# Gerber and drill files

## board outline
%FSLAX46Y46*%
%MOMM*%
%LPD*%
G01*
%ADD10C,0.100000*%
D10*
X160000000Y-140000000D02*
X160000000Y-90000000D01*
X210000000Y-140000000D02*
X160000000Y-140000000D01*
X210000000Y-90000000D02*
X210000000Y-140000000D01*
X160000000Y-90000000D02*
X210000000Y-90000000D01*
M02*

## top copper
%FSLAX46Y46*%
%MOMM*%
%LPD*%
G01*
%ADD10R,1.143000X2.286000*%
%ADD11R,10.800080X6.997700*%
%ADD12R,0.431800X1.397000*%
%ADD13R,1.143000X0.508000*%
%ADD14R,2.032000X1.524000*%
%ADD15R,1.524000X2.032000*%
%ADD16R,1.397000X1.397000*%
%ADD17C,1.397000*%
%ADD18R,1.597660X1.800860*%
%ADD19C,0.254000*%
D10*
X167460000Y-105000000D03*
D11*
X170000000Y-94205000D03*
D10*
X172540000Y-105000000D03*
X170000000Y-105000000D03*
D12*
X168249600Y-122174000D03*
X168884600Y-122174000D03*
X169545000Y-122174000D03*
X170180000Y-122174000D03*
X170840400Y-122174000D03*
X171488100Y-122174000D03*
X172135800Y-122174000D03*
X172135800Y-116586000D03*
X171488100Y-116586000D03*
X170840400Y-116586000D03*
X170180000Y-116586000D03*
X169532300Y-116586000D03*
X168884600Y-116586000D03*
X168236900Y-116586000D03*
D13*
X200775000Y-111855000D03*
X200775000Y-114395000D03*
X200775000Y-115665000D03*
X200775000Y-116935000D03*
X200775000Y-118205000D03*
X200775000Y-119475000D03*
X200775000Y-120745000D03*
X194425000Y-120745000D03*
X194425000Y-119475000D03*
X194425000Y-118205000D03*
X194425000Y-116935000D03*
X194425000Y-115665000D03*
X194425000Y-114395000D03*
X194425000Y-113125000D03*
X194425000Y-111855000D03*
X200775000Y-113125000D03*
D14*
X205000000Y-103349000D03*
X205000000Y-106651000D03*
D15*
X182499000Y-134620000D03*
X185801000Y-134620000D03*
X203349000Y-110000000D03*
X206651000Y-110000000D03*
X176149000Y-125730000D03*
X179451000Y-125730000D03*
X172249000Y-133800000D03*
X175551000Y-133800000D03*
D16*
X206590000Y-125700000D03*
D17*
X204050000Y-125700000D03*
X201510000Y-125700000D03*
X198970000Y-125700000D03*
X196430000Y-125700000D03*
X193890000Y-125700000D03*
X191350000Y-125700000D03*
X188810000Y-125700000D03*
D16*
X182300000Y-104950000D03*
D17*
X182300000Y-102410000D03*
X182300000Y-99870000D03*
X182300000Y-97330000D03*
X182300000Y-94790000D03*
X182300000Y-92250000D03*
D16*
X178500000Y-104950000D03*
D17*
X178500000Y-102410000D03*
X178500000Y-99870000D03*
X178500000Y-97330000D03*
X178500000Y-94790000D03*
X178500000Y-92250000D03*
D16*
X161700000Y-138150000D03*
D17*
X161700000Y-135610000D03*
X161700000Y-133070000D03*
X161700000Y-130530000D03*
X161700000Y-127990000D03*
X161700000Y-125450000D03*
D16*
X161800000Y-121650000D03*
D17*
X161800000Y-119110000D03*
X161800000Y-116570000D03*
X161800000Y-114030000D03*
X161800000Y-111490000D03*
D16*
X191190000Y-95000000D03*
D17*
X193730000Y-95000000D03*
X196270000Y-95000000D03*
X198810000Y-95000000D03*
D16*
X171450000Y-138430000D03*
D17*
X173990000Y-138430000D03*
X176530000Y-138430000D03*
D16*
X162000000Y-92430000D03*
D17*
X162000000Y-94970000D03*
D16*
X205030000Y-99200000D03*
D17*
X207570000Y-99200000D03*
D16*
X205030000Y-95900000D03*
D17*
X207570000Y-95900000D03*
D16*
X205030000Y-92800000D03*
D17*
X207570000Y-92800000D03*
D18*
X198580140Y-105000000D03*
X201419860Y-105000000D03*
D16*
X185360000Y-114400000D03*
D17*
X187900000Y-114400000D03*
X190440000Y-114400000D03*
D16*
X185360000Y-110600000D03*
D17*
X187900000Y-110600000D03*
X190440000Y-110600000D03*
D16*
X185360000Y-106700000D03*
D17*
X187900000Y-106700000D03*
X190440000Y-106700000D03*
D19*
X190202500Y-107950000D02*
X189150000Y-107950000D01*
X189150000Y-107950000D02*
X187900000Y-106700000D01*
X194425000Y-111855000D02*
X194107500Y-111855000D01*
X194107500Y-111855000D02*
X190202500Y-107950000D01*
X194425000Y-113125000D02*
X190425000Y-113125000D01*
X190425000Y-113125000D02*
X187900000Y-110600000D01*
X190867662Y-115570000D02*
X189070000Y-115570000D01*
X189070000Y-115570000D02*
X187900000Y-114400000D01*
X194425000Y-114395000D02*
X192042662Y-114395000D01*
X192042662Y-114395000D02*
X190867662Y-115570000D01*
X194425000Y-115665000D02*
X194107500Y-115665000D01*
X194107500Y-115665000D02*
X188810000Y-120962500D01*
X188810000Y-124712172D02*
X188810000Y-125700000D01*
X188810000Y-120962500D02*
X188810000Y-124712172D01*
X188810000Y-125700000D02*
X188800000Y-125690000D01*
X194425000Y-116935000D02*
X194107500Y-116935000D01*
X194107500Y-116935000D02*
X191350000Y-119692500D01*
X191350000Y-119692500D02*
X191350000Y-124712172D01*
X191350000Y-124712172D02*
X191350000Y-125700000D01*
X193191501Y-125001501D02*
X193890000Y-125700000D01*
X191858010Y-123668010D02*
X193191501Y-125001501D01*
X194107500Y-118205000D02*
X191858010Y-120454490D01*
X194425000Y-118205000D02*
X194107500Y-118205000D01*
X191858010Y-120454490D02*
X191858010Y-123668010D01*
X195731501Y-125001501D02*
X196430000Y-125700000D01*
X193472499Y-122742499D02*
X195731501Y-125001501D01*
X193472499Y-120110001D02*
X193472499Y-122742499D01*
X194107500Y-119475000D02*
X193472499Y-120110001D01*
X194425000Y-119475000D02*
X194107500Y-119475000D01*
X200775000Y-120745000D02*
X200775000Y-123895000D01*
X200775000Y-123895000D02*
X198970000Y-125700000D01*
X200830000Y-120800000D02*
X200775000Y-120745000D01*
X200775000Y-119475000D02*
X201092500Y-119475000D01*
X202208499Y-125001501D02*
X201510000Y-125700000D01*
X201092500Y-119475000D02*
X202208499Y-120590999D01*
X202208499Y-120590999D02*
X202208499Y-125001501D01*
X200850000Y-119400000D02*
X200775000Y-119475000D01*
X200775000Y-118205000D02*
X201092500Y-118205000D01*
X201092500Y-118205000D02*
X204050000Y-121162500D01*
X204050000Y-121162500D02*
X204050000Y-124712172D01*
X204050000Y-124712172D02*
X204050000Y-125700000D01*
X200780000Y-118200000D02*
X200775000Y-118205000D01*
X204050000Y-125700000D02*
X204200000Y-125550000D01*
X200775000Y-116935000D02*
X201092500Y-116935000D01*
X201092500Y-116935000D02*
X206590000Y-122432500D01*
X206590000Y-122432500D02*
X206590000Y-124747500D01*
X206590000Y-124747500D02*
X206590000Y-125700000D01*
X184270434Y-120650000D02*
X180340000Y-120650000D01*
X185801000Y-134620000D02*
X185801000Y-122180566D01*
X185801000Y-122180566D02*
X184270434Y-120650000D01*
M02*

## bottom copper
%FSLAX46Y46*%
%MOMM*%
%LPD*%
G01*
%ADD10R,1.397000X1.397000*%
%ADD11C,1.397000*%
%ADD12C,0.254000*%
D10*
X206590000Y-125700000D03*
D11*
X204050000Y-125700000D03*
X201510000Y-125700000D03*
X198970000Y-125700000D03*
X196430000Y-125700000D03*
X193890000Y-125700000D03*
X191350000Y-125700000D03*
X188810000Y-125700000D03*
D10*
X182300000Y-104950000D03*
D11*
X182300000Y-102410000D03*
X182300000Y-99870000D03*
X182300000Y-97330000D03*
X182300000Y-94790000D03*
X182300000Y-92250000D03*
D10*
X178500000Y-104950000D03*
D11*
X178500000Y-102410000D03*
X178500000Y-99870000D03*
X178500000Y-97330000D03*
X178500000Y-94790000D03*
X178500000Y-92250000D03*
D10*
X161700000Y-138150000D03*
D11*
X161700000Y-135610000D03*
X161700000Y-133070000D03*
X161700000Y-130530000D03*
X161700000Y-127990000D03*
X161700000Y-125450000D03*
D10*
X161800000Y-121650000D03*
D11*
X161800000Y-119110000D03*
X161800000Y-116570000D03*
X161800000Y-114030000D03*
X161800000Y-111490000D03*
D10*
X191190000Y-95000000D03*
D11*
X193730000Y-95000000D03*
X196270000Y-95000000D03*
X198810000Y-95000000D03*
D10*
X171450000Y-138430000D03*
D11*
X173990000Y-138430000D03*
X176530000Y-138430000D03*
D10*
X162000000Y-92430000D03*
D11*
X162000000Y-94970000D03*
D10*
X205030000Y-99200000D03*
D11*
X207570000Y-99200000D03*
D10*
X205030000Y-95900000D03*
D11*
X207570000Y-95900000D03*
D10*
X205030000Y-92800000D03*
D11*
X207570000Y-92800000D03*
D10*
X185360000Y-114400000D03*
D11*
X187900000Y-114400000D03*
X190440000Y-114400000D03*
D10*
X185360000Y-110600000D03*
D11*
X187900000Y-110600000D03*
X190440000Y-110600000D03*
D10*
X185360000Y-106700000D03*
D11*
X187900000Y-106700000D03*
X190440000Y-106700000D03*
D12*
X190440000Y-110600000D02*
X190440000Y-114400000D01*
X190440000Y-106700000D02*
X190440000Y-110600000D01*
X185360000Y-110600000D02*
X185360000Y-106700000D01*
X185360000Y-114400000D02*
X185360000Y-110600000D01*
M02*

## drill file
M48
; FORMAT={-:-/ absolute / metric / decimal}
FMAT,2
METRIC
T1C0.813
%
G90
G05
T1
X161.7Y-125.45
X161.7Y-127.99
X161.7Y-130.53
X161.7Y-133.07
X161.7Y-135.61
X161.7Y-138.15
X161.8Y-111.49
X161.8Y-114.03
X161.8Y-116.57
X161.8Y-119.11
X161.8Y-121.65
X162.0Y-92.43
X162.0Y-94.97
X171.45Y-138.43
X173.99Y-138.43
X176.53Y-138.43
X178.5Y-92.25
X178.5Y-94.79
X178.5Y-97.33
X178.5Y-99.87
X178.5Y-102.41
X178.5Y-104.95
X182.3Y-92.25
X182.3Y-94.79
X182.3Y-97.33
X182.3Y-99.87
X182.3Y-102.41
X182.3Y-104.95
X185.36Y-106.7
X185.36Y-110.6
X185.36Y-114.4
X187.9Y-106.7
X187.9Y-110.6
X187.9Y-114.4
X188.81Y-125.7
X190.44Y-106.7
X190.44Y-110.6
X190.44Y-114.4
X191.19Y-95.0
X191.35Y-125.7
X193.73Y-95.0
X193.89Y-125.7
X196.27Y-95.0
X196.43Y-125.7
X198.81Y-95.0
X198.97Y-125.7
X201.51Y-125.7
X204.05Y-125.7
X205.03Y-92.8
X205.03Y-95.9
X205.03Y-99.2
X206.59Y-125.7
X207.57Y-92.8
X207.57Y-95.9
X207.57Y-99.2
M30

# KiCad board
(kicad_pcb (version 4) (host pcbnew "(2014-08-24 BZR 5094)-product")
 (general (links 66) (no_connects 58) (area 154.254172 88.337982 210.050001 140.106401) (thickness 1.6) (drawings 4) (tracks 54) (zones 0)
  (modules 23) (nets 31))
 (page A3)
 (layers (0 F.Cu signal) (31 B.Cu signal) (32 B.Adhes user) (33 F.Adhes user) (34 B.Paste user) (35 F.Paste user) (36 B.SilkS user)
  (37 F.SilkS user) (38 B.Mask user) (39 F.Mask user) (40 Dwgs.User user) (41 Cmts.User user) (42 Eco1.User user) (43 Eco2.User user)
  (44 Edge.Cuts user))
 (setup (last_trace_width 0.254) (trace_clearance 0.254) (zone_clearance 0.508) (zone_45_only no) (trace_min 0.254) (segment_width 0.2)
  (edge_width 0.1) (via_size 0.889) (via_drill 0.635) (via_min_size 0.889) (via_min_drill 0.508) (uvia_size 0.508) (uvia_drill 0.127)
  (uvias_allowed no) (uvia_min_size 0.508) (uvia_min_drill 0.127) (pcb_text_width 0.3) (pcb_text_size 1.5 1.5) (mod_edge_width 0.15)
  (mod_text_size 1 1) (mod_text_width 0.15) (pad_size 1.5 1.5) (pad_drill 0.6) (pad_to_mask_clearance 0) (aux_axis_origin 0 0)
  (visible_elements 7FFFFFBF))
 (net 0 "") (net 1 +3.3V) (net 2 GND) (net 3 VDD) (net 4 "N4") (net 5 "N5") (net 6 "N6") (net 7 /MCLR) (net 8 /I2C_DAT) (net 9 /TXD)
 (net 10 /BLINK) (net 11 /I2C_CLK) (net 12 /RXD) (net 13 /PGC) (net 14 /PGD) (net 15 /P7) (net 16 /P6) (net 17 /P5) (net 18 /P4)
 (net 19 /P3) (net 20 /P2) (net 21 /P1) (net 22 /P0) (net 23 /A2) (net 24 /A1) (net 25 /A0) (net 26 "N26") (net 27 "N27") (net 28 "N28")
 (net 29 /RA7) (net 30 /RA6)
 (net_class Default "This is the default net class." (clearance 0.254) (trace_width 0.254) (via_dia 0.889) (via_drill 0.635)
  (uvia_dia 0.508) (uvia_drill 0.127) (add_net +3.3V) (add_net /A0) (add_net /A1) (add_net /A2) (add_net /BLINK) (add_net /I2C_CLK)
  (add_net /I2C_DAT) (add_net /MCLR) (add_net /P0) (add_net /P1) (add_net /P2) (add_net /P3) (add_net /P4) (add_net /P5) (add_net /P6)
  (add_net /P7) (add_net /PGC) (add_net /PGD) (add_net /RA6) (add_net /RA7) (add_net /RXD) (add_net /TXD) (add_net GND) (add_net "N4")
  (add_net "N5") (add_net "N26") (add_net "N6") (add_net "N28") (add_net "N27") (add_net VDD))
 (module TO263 (layer F.Cu) (at 170 105)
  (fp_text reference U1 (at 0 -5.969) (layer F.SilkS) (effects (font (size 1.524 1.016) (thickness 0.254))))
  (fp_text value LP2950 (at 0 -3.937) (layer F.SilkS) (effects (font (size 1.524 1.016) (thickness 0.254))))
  (pad 1 smd rect (at -2.54 0) (size 1.143 2.286) (layers F.Cu F.Paste F.Mask) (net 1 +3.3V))
  (pad 2 smd rect (at 0 -10.795) (size 10.80008 6.9977) (layers F.Cu F.Paste F.Mask) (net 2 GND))
  (pad 3 smd rect (at 2.54 0) (size 1.143 2.286) (layers F.Cu F.Paste F.Mask) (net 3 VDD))
  (pad 2 smd rect (at 0 0) (size 1.143 2.286) (layers F.Cu F.Paste F.Mask) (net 2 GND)))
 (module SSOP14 (layer F.Cu) (at 170.18 119.38)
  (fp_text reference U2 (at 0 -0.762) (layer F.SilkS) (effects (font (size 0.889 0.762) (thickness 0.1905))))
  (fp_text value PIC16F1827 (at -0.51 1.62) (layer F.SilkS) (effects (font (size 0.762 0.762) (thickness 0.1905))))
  (pad 1 smd rect (at -1.9304 2.794) (size 0.4318 1.397) (layers F.Cu F.Paste F.Mask) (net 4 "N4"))
  (pad 2 smd rect (at -1.2954 2.794) (size 0.4318 1.397) (layers F.Cu F.Paste F.Mask) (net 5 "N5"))
  (pad 3 smd rect (at -0.635 2.794) (size 0.4318 1.397) (layers F.Cu F.Paste F.Mask) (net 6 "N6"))
  (pad 4 smd rect (at 0 2.794) (size 0.4318 1.397) (layers F.Cu F.Paste F.Mask) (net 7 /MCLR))
  (pad 5 smd rect (at 0.6604 2.794) (size 0.4318 1.397) (layers F.Cu F.Paste F.Mask) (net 2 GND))
  (pad 6 smd rect (at 1.3081 2.794) (size 0.4318 1.397) (layers F.Cu F.Paste F.Mask))
  (pad 7 smd rect (at 1.9558 2.794) (size 0.4318 1.397) (layers F.Cu F.Paste F.Mask) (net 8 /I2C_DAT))
  (pad 8 smd rect (at 1.9558 -2.794) (size 0.4318 1.397) (layers F.Cu F.Paste F.Mask) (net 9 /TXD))
  (pad 9 smd rect (at 1.3081 -2.794) (size 0.4318 1.397) (layers F.Cu F.Paste F.Mask) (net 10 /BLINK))
  (pad 10 smd rect (at 0.6604 -2.794) (size 0.4318 1.397) (layers F.Cu F.Paste F.Mask) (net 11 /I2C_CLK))
  (pad 11 smd rect (at 0 -2.794) (size 0.4318 1.397) (layers F.Cu F.Paste F.Mask) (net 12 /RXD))
  (pad 12 smd rect (at -0.6477 -2.794) (size 0.4318 1.397) (layers F.Cu F.Paste F.Mask) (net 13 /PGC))
  (pad 13 smd rect (at -1.2954 -2.794) (size 0.4318 1.397) (layers F.Cu F.Paste F.Mask) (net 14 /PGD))
  (pad 14 smd rect (at -1.9431 -2.794) (size 0.4318 1.397) (layers F.Cu F.Paste F.Mask) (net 1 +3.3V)))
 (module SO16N (layer F.Cu) (at 197.6 116.3 270)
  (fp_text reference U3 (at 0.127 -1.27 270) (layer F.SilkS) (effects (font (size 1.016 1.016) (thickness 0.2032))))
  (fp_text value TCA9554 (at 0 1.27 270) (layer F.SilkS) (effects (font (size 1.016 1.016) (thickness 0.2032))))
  (pad 16 smd rect (at -4.445 -3.175 270) (size 0.508 1.143) (layers F.Cu F.Paste F.Mask) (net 1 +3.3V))
  (pad 14 smd rect (at -1.905 -3.175 270) (size 0.508 1.143) (layers F.Cu F.Paste F.Mask) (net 11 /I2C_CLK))
  (pad 13 smd rect (at -0.635 -3.175 270) (size 0.508 1.143) (layers F.Cu F.Paste F.Mask))
  (pad 12 smd rect (at 0.635 -3.175 270) (size 0.508 1.143) (layers F.Cu F.Paste F.Mask) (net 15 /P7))
  (pad 11 smd rect (at 1.905 -3.175 270) (size 0.508 1.143) (layers F.Cu F.Paste F.Mask) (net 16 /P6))
  (pad 10 smd rect (at 3.175 -3.175 270) (size 0.508 1.143) (layers F.Cu F.Paste F.Mask) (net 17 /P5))
  (pad 9 smd rect (at 4.445 -3.175 270) (size 0.508 1.143) (layers F.Cu F.Paste F.Mask) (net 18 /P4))
  (pad 8 smd rect (at 4.445 3.175 270) (size 0.508 1.143) (layers F.Cu F.Paste F.Mask) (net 2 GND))
  (pad 7 smd rect (at 3.175 3.175 270) (size 0.508 1.143) (layers F.Cu F.Paste F.Mask) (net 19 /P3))
  (pad 6 smd rect (at 1.905 3.175 270) (size 0.508 1.143) (layers F.Cu F.Paste F.Mask) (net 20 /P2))
  (pad 5 smd rect (at 0.635 3.175 270) (size 0.508 1.143) (layers F.Cu F.Paste F.Mask) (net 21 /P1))
  (pad 4 smd rect (at -0.635 3.175 270) (size 0.508 1.143) (layers F.Cu F.Paste F.Mask) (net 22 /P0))
  (pad 3 smd rect (at -1.905 3.175 270) (size 0.508 1.143) (layers F.Cu F.Paste F.Mask) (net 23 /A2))
  (pad 2 smd rect (at -3.175 3.175 270) (size 0.508 1.143) (layers F.Cu F.Paste F.Mask) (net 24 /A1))
  (pad 1 smd rect (at -4.445 3.175 270) (size 0.508 1.143) (layers F.Cu F.Paste F.Mask) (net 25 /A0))
  (pad 15 smd rect (at -3.175 -3.175 270) (size 0.508 1.143) (layers F.Cu F.Paste F.Mask) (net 8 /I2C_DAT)))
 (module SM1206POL (layer F.Cu) (at 205 105 270)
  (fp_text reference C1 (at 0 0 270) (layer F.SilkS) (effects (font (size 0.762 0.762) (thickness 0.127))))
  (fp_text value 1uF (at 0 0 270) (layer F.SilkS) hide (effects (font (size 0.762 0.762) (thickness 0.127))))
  (pad 1 smd rect (at -1.651 0 270) (size 1.524 2.032) (layers F.Cu F.Paste F.Mask) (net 3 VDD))
  (pad 2 smd rect (at 1.651 0 270) (size 1.524 2.032) (layers F.Cu F.Paste F.Mask) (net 2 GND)))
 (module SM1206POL (layer F.Cu) (at 184.15 134.62)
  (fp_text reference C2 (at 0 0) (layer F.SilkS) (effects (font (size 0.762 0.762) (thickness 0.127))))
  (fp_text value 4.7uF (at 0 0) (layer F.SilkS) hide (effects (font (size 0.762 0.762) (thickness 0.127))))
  (pad 1 smd rect (at -1.651 0) (size 1.524 2.032) (layers F.Cu F.Paste F.Mask) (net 1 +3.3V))
  (pad 2 smd rect (at 1.651 0) (size 1.524 2.032) (layers F.Cu F.Paste F.Mask) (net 2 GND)))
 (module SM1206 (layer F.Cu) (at 205 110)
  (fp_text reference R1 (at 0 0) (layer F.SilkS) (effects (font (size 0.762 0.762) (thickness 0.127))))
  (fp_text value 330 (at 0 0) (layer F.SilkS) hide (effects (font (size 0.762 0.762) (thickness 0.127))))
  (pad 1 smd rect (at -1.651 0) (size 1.524 2.032) (layers F.Cu F.Paste F.Mask) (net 10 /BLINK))
  (pad 2 smd rect (at 1.651 0) (size 1.524 2.032) (layers F.Cu F.Paste F.Mask) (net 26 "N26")))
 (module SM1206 (layer F.Cu) (at 177.8 125.73)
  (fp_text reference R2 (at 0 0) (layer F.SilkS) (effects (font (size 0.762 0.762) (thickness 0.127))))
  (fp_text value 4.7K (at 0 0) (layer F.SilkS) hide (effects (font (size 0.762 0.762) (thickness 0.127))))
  (pad 1 smd rect (at -1.651 0) (size 1.524 2.032) (layers F.Cu F.Paste F.Mask) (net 1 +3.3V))
  (pad 2 smd rect (at 1.651 0) (size 1.524 2.032) (layers F.Cu F.Paste F.Mask) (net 11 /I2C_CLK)))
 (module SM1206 (layer F.Cu) (at 173.9 133.8)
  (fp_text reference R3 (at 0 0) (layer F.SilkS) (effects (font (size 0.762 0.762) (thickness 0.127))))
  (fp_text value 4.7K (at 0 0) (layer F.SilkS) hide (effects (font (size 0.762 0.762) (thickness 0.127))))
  (pad 1 smd rect (at -1.651 0) (size 1.524 2.032) (layers F.Cu F.Paste F.Mask) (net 1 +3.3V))
  (pad 2 smd rect (at 1.651 0) (size 1.524 2.032) (layers F.Cu F.Paste F.Mask) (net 8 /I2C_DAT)))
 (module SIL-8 (layer F.Cu) (at 197.7 125.7 180)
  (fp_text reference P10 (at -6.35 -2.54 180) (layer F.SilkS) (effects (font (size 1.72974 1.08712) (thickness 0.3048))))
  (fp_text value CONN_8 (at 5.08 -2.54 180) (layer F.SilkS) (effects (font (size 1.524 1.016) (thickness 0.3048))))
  (pad 1 thru_hole rect (at -8.89 0 180) (size 1.397 1.397) (drill 0.8128) (layers *.Cu *.Mask F.SilkS) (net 15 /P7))
  (pad 2 thru_hole circle (at -6.35 0 180) (size 1.397 1.397) (drill 0.8128) (layers *.Cu *.Mask F.SilkS) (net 16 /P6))
  (pad 3 thru_hole circle (at -3.81 0 180) (size 1.397 1.397) (drill 0.8128) (layers *.Cu *.Mask F.SilkS) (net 17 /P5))
  (pad 4 thru_hole circle (at -1.27 0 180) (size 1.397 1.397) (drill 0.8128) (layers *.Cu *.Mask F.SilkS) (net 18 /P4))
  (pad 5 thru_hole circle (at 1.27 0 180) (size 1.397 1.397) (drill 0.8128) (layers *.Cu *.Mask F.SilkS) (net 19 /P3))
  (pad 6 thru_hole circle (at 3.81 0 180) (size 1.397 1.397) (drill 0.8128) (layers *.Cu *.Mask F.SilkS) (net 20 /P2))
  (pad 7 thru_hole circle (at 6.35 0 180) (size 1.397 1.397) (drill 0.8128) (layers *.Cu *.Mask F.SilkS) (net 21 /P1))
  (pad 8 thru_hole circle (at 8.89 0 180) (size 1.397 1.397) (drill 0.8128) (layers *.Cu *.Mask F.SilkS) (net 22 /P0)))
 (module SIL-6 (layer F.Cu) (at 182.3 98.6 90)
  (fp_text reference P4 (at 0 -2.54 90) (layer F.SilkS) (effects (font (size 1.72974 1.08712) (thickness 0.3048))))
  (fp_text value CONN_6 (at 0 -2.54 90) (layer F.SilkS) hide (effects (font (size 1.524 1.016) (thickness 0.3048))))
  (pad 1 thru_hole rect (at -6.35 0 90) (size 1.397 1.397) (drill 0.8128) (layers *.Cu *.Mask F.SilkS) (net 1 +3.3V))
  (pad 2 thru_hole circle (at -3.81 0 90) (size 1.397 1.397) (drill 0.8128) (layers *.Cu *.Mask F.SilkS) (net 1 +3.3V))
  (pad 3 thru_hole circle (at -1.27 0 90) (size 1.397 1.397) (drill 0.8128) (layers *.Cu *.Mask F.SilkS) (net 1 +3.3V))
  (pad 4 thru_hole circle (at 1.27 0 90) (size 1.397 1.397) (drill 0.8128) (layers *.Cu *.Mask F.SilkS) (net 1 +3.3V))
  (pad 5 thru_hole circle (at 3.81 0 90) (size 1.397 1.397) (drill 0.8128) (layers *.Cu *.Mask F.SilkS) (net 1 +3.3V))
  (pad 6 thru_hole circle (at 6.35 0 90) (size 1.397 1.397) (drill 0.8128) (layers *.Cu *.Mask F.SilkS) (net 1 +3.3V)))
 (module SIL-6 (layer F.Cu) (at 178.5 98.6 90)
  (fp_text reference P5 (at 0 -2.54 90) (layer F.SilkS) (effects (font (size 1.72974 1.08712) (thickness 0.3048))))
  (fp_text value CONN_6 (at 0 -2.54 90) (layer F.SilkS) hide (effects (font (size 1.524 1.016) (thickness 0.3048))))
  (pad 1 thru_hole rect (at -6.35 0 90) (size 1.397 1.397) (drill 0.8128) (layers *.Cu *.Mask F.SilkS) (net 2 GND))
  (pad 2 thru_hole circle (at -3.81 0 90) (size 1.397 1.397) (drill 0.8128) (layers *.Cu *.Mask F.SilkS) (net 2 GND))
  (pad 3 thru_hole circle (at -1.27 0 90) (size 1.397 1.397) (drill 0.8128) (layers *.Cu *.Mask F.SilkS) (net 2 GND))
  (pad 4 thru_hole circle (at 1.27 0 90) (size 1.397 1.397) (drill 0.8128) (layers *.Cu *.Mask F.SilkS) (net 2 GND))
  (pad 5 thru_hole circle (at 3.81 0 90) (size 1.397 1.397) (drill 0.8128) (layers *.Cu *.Mask F.SilkS) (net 2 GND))
  (pad 6 thru_hole circle (at 6.35 0 90) (size 1.397 1.397) (drill 0.8128) (layers *.Cu *.Mask F.SilkS) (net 2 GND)))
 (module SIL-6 (layer F.Cu) (at 161.7 131.8 90)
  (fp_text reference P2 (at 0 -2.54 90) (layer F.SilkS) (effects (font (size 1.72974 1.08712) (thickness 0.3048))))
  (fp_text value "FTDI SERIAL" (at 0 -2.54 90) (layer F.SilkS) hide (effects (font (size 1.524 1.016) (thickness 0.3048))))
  (pad 1 thru_hole rect (at -6.35 0 90) (size 1.397 1.397) (drill 0.8128) (layers *.Cu *.Mask F.SilkS) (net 2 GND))
  (pad 2 thru_hole circle (at -3.81 0 90) (size 1.397 1.397) (drill 0.8128) (layers *.Cu *.Mask F.SilkS))
  (pad 3 thru_hole circle (at -1.27 0 90) (size 1.397 1.397) (drill 0.8128) (layers *.Cu *.Mask F.SilkS) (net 3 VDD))
  (pad 4 thru_hole circle (at 1.27 0 90) (size 1.397 1.397) (drill 0.8128) (layers *.Cu *.Mask F.SilkS) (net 9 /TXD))
  (pad 5 thru_hole circle (at 3.81 0 90) (size 1.397 1.397) (drill 0.8128) (layers *.Cu *.Mask F.SilkS) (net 12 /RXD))
  (pad 6 thru_hole circle (at 6.35 0 90) (size 1.397 1.397) (drill 0.8128) (layers *.Cu *.Mask F.SilkS)))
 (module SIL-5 (layer F.Cu) (at 161.8 115.3 90)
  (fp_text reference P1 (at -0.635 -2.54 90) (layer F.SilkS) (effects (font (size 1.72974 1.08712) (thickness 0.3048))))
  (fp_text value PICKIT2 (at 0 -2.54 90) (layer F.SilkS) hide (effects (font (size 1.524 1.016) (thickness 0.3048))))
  (pad 1 thru_hole rect (at -6.35 0 90) (size 1.397 1.397) (drill 0.8128) (layers *.Cu *.Mask F.SilkS) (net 13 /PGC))
  (pad 2 thru_hole circle (at -3.81 0 90) (size 1.397 1.397) (drill 0.8128) (layers *.Cu *.Mask F.SilkS) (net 14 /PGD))
  (pad 3 thru_hole circle (at -1.27 0 90) (size 1.397 1.397) (drill 0.8128) (layers *.Cu *.Mask F.SilkS) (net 2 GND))
  (pad 4 thru_hole circle (at 1.27 0 90) (size 1.397 1.397) (drill 0.8128) (layers *.Cu *.Mask F.SilkS) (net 3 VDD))
  (pad 5 thru_hole circle (at 3.81 0 90) (size 1.397 1.397) (drill 0.8128) (layers *.Cu *.Mask F.SilkS) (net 7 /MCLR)))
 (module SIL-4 (layer F.Cu) (at 195 95)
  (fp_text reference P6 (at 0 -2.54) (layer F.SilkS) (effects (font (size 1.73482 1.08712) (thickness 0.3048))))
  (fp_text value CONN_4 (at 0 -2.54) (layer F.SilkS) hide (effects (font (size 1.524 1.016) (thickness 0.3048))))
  (pad 1 thru_hole rect (at -3.81 0) (size 1.397 1.397) (drill 0.8128) (layers *.Cu *.Mask F.SilkS) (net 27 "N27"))
  (pad 2 thru_hole circle (at -1.27 0) (size 1.397 1.397) (drill 0.8128) (layers *.Cu *.Mask F.SilkS) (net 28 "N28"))
  (pad 3 thru_hole circle (at 1.27 0) (size 1.397 1.397) (drill 0.8128) (layers *.Cu *.Mask F.SilkS) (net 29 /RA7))
  (pad 4 thru_hole circle (at 3.81 0) (size 1.397 1.397) (drill 0.8128) (layers *.Cu *.Mask F.SilkS) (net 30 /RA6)))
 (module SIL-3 (layer F.Cu) (at 173.99 138.43)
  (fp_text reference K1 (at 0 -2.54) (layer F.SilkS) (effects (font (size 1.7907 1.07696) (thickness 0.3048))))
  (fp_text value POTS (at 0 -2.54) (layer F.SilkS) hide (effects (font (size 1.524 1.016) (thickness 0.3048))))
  (pad 1 thru_hole rect (at -2.54 0) (size 1.397 1.397) (drill 0.8128) (layers *.Cu *.Mask F.SilkS) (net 6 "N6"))
  (pad 2 thru_hole circle (at 0 0) (size 1.397 1.397) (drill 0.8128) (layers *.Cu *.Mask F.SilkS) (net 5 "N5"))
  (pad 3 thru_hole circle (at 2.54 0) (size 1.397 1.397) (drill 0.8128) (layers *.Cu *.Mask F.SilkS) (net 4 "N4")))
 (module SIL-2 (layer F.Cu) (at 162 93.7 270)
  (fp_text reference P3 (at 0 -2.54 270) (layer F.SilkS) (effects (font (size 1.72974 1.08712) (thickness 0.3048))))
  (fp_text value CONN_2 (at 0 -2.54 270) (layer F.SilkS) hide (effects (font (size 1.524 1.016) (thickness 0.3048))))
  (pad 1 thru_hole rect (at -1.27 0 270) (size 1.397 1.397) (drill 0.8128) (layers *.Cu *.Mask F.SilkS) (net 2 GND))
  (pad 2 thru_hole circle (at 1.27 0 270) (size 1.397 1.397) (drill 0.8128) (layers *.Cu *.Mask F.SilkS) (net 3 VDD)))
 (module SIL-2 (layer F.Cu) (at 206.3 99.2)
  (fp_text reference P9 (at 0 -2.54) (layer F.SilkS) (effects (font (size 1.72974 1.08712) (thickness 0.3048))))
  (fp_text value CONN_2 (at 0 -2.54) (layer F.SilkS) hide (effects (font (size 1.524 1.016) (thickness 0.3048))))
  (pad 1 thru_hole rect (at -1.27 0) (size 1.397 1.397) (drill 0.8128) (layers *.Cu *.Mask F.SilkS) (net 11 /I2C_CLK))
  (pad 2 thru_hole circle (at 1.27 0) (size 1.397 1.397) (drill 0.8128) (layers *.Cu *.Mask F.SilkS) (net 8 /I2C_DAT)))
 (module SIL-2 (layer F.Cu) (at 206.3 95.9)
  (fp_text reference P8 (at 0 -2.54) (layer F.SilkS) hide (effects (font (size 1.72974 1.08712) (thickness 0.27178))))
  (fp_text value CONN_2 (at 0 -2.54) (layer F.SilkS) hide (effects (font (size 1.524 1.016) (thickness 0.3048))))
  (pad 1 thru_hole rect (at -1.27 0) (size 1.397 1.397) (drill 0.8128) (layers *.Cu *.Mask F.SilkS) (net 11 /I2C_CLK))
  (pad 2 thru_hole circle (at 1.27 0) (size 1.397 1.397) (drill 0.8128) (layers *.Cu *.Mask F.SilkS) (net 8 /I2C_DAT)))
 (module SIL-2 (layer F.Cu) (at 206.3 92.8)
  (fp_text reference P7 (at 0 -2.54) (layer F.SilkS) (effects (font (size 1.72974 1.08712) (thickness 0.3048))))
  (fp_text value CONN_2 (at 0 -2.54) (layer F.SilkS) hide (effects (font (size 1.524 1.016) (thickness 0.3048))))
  (pad 1 thru_hole rect (at -1.27 0) (size 1.397 1.397) (drill 0.8128) (layers *.Cu *.Mask F.SilkS))
  (pad 2 thru_hole circle (at 1.27 0) (size 1.397 1.397) (drill 0.8128) (layers *.Cu *.Mask F.SilkS) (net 8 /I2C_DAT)))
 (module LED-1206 (layer F.Cu) (at 200 105)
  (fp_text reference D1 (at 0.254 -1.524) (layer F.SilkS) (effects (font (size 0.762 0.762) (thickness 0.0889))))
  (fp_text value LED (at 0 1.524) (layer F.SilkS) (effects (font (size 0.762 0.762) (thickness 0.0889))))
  (pad 1 smd rect (at -1.41986 0) (size 1.59766 1.80086) (layers F.Cu F.Paste F.Mask) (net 26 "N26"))
  (pad 2 smd rect (at 1.41986 0) (size 1.59766 1.80086) (layers F.Cu F.Paste F.Mask) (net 2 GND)))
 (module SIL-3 (layer F.Cu) (at 187.9 114.4)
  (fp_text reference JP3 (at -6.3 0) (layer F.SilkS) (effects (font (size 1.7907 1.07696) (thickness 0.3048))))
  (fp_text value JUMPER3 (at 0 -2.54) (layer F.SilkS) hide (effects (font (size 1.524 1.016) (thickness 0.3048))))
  (pad 1 thru_hole rect (at -2.54 0) (size 1.397 1.397) (drill 0.8128) (layers *.Cu *.Mask F.SilkS) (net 2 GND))
  (pad 2 thru_hole circle (at 0 0) (size 1.397 1.397) (drill 0.8128) (layers *.Cu *.Mask F.SilkS) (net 23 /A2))
  (pad 3 thru_hole circle (at 2.54 0) (size 1.397 1.397) (drill 0.8128) (layers *.Cu *.Mask F.SilkS) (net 1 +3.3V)))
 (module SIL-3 (layer F.Cu) (at 187.9 110.6)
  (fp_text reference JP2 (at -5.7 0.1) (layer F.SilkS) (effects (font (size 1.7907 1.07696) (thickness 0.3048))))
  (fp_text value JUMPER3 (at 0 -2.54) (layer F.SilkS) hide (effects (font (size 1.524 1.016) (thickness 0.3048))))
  (pad 1 thru_hole rect (at -2.54 0) (size 1.397 1.397) (drill 0.8128) (layers *.Cu *.Mask F.SilkS) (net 2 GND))
  (pad 2 thru_hole circle (at 0 0) (size 1.397 1.397) (drill 0.8128) (layers *.Cu *.Mask F.SilkS) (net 24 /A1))
  (pad 3 thru_hole circle (at 2.54 0) (size 1.397 1.397) (drill 0.8128) (layers *.Cu *.Mask F.SilkS) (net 1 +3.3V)))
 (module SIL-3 (layer F.Cu) (at 187.9 106.7)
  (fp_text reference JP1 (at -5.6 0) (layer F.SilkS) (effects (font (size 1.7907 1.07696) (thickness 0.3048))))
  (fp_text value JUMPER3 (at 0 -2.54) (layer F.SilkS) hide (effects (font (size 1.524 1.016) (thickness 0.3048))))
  (pad 1 thru_hole rect (at -2.54 0) (size 1.397 1.397) (drill 0.8128) (layers *.Cu *.Mask F.SilkS) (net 2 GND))
  (pad 2 thru_hole circle (at 0 0) (size 1.397 1.397) (drill 0.8128) (layers *.Cu *.Mask F.SilkS) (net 25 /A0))
  (pad 3 thru_hole circle (at 2.54 0) (size 1.397 1.397) (drill 0.8128) (layers *.Cu *.Mask F.SilkS) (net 1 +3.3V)))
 (gr_line (start 160 140) (end 160 90) (angle 90) (layer Edge.Cuts) (width 0.1))
 (gr_line (start 210 140) (end 160 140) (angle 90) (layer Edge.Cuts) (width 0.1))
 (gr_line (start 210 90) (end 210 140) (angle 90) (layer Edge.Cuts) (width 0.1))
 (gr_line (start 160 90) (end 210 90) (angle 90) (layer Edge.Cuts) (width 0.1))
 (segment (start 190.44 110.6) (end 190.44 114.4) (width 0.254) (layer B.Cu) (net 1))
 (segment (start 190.44 106.7) (end 190.44 110.6) (width 0.254) (layer B.Cu) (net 1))
 (segment (start 190.2025 107.95) (end 189.15 107.95) (width 0.254) (layer F.Cu) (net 25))
 (segment (start 189.15 107.95) (end 187.9 106.7) (width 0.254) (layer F.Cu) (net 25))
 (segment (start 194.425 111.855) (end 194.1075 111.855) (width 0.254) (layer F.Cu) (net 25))
 (segment (start 194.1075 111.855) (end 190.2025 107.95) (width 0.254) (layer F.Cu) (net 25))
 (segment (start 194.425 113.125) (end 190.425 113.125) (width 0.254) (layer F.Cu) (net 24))
 (segment (start 190.425 113.125) (end 187.9 110.6) (width 0.254) (layer F.Cu) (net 24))
 (segment (start 190.867662 115.57) (end 189.07 115.57) (width 0.254) (layer F.Cu) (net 23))
 (segment (start 189.07 115.57) (end 187.9 114.4) (width 0.254) (layer F.Cu) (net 23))
 (segment (start 194.425 114.395) (end 192.042662 114.395) (width 0.254) (layer F.Cu) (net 23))
 (segment (start 192.042662 114.395) (end 190.867662 115.57) (width 0.254) (layer F.Cu) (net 23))
 (segment (start 194.425 115.665) (end 194.1075 115.665) (width 0.254) (layer F.Cu) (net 22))
 (segment (start 194.1075 115.665) (end 188.81 120.9625) (width 0.254) (layer F.Cu) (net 22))
 (segment (start 188.81 124.712172) (end 188.81 125.7) (width 0.254) (layer F.Cu) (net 22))
 (segment (start 188.81 120.9625) (end 188.81 124.712172) (width 0.254) (layer F.Cu) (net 22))
 (segment (start 188.81 125.7) (end 188.8 125.69) (width 0.254) (layer F.Cu) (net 22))
 (segment (start 194.425 116.935) (end 194.1075 116.935) (width 0.254) (layer F.Cu) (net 21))
 (segment (start 194.1075 116.935) (end 191.35 119.6925) (width 0.254) (layer F.Cu) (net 21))
 (segment (start 191.35 119.6925) (end 191.35 124.712172) (width 0.254) (layer F.Cu) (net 21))
 (segment (start 191.35 124.712172) (end 191.35 125.7) (width 0.254) (layer F.Cu) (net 21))
 (segment (start 193.191501 125.001501) (end 193.89 125.7) (width 0.254) (layer F.Cu) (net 20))
 (segment (start 191.85801 123.66801) (end 193.191501 125.001501) (width 0.254) (layer F.Cu) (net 20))
 (segment (start 194.1075 118.205) (end 191.85801 120.45449) (width 0.254) (layer F.Cu) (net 20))
 (segment (start 194.425 118.205) (end 194.1075 118.205) (width 0.254) (layer F.Cu) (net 20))
 (segment (start 191.85801 120.45449) (end 191.85801 123.66801) (width 0.254) (layer F.Cu) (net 20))
 (segment (start 195.731501 125.001501) (end 196.43 125.7) (width 0.254) (layer F.Cu) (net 19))
 (segment (start 193.472499 122.742499) (end 195.731501 125.001501) (width 0.254) (layer F.Cu) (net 19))
 (segment (start 193.472499 120.110001) (end 193.472499 122.742499) (width 0.254) (layer F.Cu) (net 19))
 (segment (start 194.1075 119.475) (end 193.472499 120.110001) (width 0.254) (layer F.Cu) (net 19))
 (segment (start 194.425 119.475) (end 194.1075 119.475) (width 0.254) (layer F.Cu) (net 19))
 (segment (start 200.775 120.745) (end 200.775 123.895) (width 0.254) (layer F.Cu) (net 18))
 (segment (start 200.775 123.895) (end 198.97 125.7) (width 0.254) (layer F.Cu) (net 18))
 (segment (start 200.83 120.8) (end 200.775 120.745) (width 0.254) (layer F.Cu) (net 18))
 (segment (start 200.775 119.475) (end 201.0925 119.475) (width 0.254) (layer F.Cu) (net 17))
 (segment (start 202.208499 125.001501) (end 201.51 125.7) (width 0.254) (layer F.Cu) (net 17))
 (segment (start 201.0925 119.475) (end 202.208499 120.590999) (width 0.254) (layer F.Cu) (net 17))
 (segment (start 202.208499 120.590999) (end 202.208499 125.001501) (width 0.254) (layer F.Cu) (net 17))
 (segment (start 200.85 119.4) (end 200.775 119.475) (width 0.254) (layer F.Cu) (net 17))
 (segment (start 200.775 118.205) (end 201.0925 118.205) (width 0.254) (layer F.Cu) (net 16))
 (segment (start 201.0925 118.205) (end 204.05 121.1625) (width 0.254) (layer F.Cu) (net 16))
 (segment (start 204.05 121.1625) (end 204.05 124.712172) (width 0.254) (layer F.Cu) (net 16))
 (segment (start 204.05 124.712172) (end 204.05 125.7) (width 0.254) (layer F.Cu) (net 16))
 (segment (start 200.78 118.2) (end 200.775 118.205) (width 0.254) (layer F.Cu) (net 16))
 (segment (start 204.05 125.7) (end 204.2 125.55) (width 0.254) (layer F.Cu) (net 16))
 (segment (start 200.775 116.935) (end 201.0925 116.935) (width 0.254) (layer F.Cu) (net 15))
 (segment (start 201.0925 116.935) (end 206.59 122.4325) (width 0.254) (layer F.Cu) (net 15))
 (segment (start 206.59 122.4325) (end 206.59 124.7475) (width 0.254) (layer F.Cu) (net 15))
 (segment (start 206.59 124.7475) (end 206.59 125.7) (width 0.254) (layer F.Cu) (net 15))
 (segment (start 184.270434 120.65) (end 180.34 120.65) (width 0.254) (layer F.Cu) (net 2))
 (segment (start 185.801 134.62) (end 185.801 122.180566) (width 0.254) (layer F.Cu) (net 2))
 (segment (start 185.801 122.180566) (end 184.270434 120.65) (width 0.254) (layer F.Cu) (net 2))
 (segment (start 185.36 110.6) (end 185.36 106.7) (width 0.254) (layer B.Cu) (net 2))
 (segment (start 185.36 114.4) (end 185.36 110.6) (width 0.254) (layer B.Cu) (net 2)))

